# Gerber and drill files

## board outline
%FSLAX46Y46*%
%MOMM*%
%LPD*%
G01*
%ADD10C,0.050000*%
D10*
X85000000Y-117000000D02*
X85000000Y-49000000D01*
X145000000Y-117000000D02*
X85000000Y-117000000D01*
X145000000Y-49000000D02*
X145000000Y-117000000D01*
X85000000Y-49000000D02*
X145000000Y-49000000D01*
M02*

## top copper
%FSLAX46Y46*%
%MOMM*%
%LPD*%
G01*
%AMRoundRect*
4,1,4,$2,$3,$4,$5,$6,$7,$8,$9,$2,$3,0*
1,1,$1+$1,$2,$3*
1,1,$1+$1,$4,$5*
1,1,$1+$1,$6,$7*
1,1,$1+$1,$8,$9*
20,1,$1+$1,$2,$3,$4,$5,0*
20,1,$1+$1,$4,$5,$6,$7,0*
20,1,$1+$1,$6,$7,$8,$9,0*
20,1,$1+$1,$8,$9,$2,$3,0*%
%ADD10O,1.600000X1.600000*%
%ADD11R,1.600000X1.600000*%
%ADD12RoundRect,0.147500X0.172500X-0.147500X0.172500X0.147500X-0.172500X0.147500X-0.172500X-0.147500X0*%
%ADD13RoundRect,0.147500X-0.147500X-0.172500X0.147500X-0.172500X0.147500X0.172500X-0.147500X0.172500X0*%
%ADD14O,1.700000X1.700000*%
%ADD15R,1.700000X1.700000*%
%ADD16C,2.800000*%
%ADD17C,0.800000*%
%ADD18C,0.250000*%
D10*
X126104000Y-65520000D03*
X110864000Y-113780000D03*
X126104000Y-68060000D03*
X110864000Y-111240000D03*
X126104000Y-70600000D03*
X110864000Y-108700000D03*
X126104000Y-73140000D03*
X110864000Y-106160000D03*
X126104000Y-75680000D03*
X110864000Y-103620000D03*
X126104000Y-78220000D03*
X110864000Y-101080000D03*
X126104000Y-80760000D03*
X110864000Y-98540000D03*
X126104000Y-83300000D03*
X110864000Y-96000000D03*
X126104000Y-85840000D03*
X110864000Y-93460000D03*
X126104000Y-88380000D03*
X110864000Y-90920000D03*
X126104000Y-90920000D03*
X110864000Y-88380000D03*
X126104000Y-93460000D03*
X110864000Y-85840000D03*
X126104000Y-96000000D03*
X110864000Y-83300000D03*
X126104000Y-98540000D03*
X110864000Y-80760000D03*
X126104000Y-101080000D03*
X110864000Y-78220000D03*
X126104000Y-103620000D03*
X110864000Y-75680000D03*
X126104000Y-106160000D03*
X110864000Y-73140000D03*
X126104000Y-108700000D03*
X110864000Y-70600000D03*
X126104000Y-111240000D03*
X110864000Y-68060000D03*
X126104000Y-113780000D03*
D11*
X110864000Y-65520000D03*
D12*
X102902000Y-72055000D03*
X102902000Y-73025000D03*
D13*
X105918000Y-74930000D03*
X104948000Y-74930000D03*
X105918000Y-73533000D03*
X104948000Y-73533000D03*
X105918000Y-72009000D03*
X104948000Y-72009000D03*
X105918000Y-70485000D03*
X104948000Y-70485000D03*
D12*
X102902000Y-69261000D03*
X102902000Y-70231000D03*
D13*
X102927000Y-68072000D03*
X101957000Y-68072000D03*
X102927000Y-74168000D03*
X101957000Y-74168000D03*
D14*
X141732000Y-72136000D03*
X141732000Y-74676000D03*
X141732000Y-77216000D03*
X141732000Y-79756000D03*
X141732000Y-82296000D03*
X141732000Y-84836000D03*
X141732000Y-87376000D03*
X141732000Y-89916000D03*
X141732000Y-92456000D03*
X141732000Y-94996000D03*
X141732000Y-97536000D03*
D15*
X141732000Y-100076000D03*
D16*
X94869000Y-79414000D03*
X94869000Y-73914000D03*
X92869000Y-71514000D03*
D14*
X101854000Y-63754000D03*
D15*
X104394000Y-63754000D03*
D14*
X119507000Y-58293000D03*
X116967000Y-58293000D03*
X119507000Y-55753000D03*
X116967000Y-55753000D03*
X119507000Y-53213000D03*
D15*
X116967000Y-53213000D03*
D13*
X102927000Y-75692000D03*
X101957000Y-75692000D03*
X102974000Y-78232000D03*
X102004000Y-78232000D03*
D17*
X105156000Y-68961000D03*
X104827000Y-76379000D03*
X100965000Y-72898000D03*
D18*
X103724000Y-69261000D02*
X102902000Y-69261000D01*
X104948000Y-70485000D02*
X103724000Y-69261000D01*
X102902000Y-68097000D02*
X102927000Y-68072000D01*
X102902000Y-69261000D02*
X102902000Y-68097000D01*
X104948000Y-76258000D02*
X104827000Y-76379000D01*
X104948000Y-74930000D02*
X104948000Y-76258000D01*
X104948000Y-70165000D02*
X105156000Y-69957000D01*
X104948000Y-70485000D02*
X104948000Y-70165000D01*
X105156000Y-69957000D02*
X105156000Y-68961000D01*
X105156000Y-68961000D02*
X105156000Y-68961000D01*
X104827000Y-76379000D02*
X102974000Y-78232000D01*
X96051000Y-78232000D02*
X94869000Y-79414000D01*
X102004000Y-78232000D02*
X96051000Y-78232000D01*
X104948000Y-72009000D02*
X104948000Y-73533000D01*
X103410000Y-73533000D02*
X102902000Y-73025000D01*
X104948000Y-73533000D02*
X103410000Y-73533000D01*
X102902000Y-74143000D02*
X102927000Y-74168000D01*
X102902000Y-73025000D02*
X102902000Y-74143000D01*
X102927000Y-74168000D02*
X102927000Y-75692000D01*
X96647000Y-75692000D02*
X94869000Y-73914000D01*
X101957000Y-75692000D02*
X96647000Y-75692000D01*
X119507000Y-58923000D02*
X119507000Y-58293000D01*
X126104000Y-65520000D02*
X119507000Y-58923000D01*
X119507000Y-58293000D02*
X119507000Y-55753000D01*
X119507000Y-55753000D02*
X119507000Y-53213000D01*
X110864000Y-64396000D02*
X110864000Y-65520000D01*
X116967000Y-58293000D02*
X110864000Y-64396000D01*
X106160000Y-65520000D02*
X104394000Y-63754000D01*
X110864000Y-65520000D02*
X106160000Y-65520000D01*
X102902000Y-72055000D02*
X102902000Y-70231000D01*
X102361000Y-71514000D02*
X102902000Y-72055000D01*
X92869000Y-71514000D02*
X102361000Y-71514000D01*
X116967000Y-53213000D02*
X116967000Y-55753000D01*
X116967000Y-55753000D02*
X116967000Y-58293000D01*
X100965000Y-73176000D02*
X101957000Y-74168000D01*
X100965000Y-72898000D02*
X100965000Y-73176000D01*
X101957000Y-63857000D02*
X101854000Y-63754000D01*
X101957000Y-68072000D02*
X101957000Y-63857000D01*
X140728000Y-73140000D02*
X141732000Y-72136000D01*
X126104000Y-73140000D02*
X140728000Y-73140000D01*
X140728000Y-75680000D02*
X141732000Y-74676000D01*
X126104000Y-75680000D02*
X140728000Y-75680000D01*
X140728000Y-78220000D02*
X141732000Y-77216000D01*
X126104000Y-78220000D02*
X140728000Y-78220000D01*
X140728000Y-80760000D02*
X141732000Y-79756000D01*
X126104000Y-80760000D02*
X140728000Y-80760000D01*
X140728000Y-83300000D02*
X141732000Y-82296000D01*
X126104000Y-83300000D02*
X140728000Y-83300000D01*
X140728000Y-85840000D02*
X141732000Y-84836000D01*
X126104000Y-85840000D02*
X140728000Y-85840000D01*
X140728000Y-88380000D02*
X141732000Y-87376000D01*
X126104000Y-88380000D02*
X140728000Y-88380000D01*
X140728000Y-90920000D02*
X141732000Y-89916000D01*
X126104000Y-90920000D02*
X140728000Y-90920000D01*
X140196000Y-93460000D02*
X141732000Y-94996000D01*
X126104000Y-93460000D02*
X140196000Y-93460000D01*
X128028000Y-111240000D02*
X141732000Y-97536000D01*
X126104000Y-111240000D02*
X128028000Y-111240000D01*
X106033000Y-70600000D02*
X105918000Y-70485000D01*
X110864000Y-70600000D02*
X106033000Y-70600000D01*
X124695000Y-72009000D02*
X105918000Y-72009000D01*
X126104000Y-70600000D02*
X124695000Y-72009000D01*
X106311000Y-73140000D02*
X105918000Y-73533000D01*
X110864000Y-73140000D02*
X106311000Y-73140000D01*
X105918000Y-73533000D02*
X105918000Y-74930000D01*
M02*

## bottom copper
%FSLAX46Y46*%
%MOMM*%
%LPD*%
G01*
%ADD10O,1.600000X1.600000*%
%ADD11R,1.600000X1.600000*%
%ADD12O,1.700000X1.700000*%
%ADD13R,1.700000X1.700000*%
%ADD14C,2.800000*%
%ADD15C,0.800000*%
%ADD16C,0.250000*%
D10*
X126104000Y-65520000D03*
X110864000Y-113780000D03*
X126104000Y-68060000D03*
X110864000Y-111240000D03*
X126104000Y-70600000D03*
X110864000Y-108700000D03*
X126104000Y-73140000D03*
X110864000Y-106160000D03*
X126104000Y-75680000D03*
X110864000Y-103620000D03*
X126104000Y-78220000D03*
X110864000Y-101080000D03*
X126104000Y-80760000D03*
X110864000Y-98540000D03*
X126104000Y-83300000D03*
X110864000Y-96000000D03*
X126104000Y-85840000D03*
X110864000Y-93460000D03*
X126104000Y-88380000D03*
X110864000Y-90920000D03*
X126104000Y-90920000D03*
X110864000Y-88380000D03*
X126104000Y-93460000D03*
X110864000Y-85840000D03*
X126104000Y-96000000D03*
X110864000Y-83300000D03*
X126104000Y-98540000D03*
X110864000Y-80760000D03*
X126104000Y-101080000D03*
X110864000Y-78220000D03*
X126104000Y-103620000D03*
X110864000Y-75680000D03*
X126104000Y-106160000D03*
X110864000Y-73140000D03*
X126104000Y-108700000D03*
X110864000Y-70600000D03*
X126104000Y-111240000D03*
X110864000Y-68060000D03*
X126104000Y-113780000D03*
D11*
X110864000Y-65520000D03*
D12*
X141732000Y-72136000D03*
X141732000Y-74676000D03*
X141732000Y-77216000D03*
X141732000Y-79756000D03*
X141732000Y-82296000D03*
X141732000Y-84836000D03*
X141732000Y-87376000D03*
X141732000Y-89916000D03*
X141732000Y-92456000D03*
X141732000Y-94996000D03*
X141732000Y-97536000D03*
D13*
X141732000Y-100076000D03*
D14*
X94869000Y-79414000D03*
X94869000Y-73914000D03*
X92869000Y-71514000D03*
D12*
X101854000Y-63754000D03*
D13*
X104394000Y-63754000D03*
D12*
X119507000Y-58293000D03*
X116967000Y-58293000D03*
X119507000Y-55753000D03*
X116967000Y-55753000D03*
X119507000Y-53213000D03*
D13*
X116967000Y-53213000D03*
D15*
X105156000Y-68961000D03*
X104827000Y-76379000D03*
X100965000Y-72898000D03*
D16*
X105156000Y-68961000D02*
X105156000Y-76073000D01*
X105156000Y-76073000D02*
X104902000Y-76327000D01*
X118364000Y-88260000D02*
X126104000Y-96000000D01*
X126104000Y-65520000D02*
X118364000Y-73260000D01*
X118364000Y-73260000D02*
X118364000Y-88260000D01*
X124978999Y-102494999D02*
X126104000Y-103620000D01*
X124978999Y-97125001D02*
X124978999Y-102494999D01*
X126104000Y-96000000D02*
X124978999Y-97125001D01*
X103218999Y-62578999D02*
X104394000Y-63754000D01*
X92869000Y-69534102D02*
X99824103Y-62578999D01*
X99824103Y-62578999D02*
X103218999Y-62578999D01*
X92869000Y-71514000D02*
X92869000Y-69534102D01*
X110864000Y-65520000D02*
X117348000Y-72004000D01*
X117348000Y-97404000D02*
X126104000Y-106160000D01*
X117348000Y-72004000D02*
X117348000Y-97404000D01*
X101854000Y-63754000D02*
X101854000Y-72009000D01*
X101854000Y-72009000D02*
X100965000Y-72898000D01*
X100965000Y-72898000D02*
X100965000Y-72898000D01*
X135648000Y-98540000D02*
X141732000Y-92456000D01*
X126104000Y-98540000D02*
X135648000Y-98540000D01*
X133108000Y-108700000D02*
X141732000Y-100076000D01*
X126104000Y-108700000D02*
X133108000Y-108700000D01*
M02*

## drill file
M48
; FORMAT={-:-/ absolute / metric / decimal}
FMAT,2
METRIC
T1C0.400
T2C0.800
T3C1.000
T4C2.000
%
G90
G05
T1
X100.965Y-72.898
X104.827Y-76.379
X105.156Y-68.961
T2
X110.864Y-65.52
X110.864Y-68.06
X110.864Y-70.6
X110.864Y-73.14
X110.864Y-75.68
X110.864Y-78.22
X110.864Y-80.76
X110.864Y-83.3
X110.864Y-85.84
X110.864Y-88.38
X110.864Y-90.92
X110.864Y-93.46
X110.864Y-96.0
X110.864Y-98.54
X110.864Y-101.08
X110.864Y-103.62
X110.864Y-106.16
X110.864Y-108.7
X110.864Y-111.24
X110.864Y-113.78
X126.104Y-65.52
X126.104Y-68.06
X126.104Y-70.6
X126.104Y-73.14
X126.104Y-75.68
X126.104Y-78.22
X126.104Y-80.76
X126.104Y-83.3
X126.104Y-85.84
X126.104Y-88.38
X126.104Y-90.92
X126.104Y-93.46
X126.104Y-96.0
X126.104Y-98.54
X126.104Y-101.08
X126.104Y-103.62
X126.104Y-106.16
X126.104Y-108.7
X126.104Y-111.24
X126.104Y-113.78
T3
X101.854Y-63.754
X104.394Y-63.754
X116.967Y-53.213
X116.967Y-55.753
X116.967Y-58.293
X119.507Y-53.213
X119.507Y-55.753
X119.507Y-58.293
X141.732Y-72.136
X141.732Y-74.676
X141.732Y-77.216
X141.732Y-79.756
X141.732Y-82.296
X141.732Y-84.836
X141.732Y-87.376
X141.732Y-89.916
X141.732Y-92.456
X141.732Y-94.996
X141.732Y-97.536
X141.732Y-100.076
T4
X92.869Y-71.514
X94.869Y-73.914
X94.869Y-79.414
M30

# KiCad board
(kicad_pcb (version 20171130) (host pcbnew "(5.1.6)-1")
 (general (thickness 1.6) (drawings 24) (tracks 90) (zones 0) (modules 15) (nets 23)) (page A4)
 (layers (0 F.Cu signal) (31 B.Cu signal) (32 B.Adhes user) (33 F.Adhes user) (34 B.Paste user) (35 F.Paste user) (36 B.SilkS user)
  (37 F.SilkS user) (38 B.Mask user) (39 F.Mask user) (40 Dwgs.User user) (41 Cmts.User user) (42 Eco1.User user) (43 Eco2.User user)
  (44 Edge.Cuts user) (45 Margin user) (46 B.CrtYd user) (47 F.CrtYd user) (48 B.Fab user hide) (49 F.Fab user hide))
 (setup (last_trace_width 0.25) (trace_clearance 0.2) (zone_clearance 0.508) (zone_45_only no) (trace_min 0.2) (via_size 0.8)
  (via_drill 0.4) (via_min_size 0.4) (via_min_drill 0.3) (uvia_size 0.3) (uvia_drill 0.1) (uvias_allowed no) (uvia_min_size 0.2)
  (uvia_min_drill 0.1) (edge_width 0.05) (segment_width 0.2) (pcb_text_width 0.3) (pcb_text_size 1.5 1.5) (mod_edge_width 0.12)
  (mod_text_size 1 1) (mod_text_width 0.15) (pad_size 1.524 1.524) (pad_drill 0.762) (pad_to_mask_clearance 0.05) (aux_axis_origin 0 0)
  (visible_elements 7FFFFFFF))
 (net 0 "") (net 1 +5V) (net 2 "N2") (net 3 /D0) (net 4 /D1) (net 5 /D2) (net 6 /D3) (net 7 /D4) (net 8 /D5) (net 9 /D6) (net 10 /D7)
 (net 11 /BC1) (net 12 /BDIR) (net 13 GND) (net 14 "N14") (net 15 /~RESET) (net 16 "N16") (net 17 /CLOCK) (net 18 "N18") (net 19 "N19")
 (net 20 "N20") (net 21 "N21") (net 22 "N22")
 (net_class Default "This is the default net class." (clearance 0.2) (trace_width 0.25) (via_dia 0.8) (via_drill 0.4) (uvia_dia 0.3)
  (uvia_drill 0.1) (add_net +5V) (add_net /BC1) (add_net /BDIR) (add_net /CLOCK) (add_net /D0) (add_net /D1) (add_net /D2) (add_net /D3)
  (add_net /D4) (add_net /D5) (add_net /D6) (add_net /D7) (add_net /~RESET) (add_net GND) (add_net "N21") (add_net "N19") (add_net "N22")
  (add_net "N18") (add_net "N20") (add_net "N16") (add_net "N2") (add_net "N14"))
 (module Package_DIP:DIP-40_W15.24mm (layer F.Cu) (at 110.864 65.52)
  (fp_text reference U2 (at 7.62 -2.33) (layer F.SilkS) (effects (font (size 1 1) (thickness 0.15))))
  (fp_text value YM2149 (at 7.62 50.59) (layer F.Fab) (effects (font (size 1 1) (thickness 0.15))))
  (pad 40 thru_hole oval (at 15.24 0) (size 1.6 1.6) (drill 0.8) (layers *.Cu *.Mask) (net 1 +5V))
  (pad 20 thru_hole oval (at 0 48.26) (size 1.6 1.6) (drill 0.8) (layers *.Cu *.Mask))
  (pad 39 thru_hole oval (at 15.24 2.54) (size 1.6 1.6) (drill 0.8) (layers *.Cu *.Mask))
  (pad 19 thru_hole oval (at 0 45.72) (size 1.6 1.6) (drill 0.8) (layers *.Cu *.Mask))
  (pad 38 thru_hole oval (at 15.24 5.08) (size 1.6 1.6) (drill 0.8) (layers *.Cu *.Mask) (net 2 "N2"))
  (pad 18 thru_hole oval (at 0 43.18) (size 1.6 1.6) (drill 0.8) (layers *.Cu *.Mask))
  (pad 37 thru_hole oval (at 15.24 7.62) (size 1.6 1.6) (drill 0.8) (layers *.Cu *.Mask) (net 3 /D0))
  (pad 17 thru_hole oval (at 0 40.64) (size 1.6 1.6) (drill 0.8) (layers *.Cu *.Mask))
  (pad 36 thru_hole oval (at 15.24 10.16) (size 1.6 1.6) (drill 0.8) (layers *.Cu *.Mask) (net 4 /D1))
  (pad 16 thru_hole oval (at 0 38.1) (size 1.6 1.6) (drill 0.8) (layers *.Cu *.Mask))
  (pad 35 thru_hole oval (at 15.24 12.7) (size 1.6 1.6) (drill 0.8) (layers *.Cu *.Mask) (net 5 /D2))
  (pad 15 thru_hole oval (at 0 35.56) (size 1.6 1.6) (drill 0.8) (layers *.Cu *.Mask))
  (pad 34 thru_hole oval (at 15.24 15.24) (size 1.6 1.6) (drill 0.8) (layers *.Cu *.Mask) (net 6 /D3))
  (pad 14 thru_hole oval (at 0 33.02) (size 1.6 1.6) (drill 0.8) (layers *.Cu *.Mask))
  (pad 33 thru_hole oval (at 15.24 17.78) (size 1.6 1.6) (drill 0.8) (layers *.Cu *.Mask) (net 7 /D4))
  (pad 13 thru_hole oval (at 0 30.48) (size 1.6 1.6) (drill 0.8) (layers *.Cu *.Mask))
  (pad 32 thru_hole oval (at 15.24 20.32) (size 1.6 1.6) (drill 0.8) (layers *.Cu *.Mask) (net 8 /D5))
  (pad 12 thru_hole oval (at 0 27.94) (size 1.6 1.6) (drill 0.8) (layers *.Cu *.Mask))
  (pad 31 thru_hole oval (at 15.24 22.86) (size 1.6 1.6) (drill 0.8) (layers *.Cu *.Mask) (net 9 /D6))
  (pad 11 thru_hole oval (at 0 25.4) (size 1.6 1.6) (drill 0.8) (layers *.Cu *.Mask))
  (pad 30 thru_hole oval (at 15.24 25.4) (size 1.6 1.6) (drill 0.8) (layers *.Cu *.Mask) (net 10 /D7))
  (pad 10 thru_hole oval (at 0 22.86) (size 1.6 1.6) (drill 0.8) (layers *.Cu *.Mask))
  (pad 29 thru_hole oval (at 15.24 27.94) (size 1.6 1.6) (drill 0.8) (layers *.Cu *.Mask) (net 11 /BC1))
  (pad 9 thru_hole oval (at 0 20.32) (size 1.6 1.6) (drill 0.8) (layers *.Cu *.Mask))
  (pad 28 thru_hole oval (at 15.24 30.48) (size 1.6 1.6) (drill 0.8) (layers *.Cu *.Mask) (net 1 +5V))
  (pad 8 thru_hole oval (at 0 17.78) (size 1.6 1.6) (drill 0.8) (layers *.Cu *.Mask))
  (pad 27 thru_hole oval (at 15.24 33.02) (size 1.6 1.6) (drill 0.8) (layers *.Cu *.Mask) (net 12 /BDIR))
  (pad 7 thru_hole oval (at 0 15.24) (size 1.6 1.6) (drill 0.8) (layers *.Cu *.Mask))
  (pad 26 thru_hole oval (at 15.24 35.56) (size 1.6 1.6) (drill 0.8) (layers *.Cu *.Mask))
  (pad 6 thru_hole oval (at 0 12.7) (size 1.6 1.6) (drill 0.8) (layers *.Cu *.Mask))
  (pad 25 thru_hole oval (at 15.24 38.1) (size 1.6 1.6) (drill 0.8) (layers *.Cu *.Mask) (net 1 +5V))
  (pad 5 thru_hole oval (at 0 10.16) (size 1.6 1.6) (drill 0.8) (layers *.Cu *.Mask))
  (pad 24 thru_hole oval (at 15.24 40.64) (size 1.6 1.6) (drill 0.8) (layers *.Cu *.Mask) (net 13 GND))
  (pad 4 thru_hole oval (at 0 7.62) (size 1.6 1.6) (drill 0.8) (layers *.Cu *.Mask) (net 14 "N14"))
  (pad 23 thru_hole oval (at 15.24 43.18) (size 1.6 1.6) (drill 0.8) (layers *.Cu *.Mask) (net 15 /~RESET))
  (pad 3 thru_hole oval (at 0 5.08) (size 1.6 1.6) (drill 0.8) (layers *.Cu *.Mask) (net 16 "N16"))
  (pad 22 thru_hole oval (at 15.24 45.72) (size 1.6 1.6) (drill 0.8) (layers *.Cu *.Mask) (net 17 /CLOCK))
  (pad 2 thru_hole oval (at 0 2.54) (size 1.6 1.6) (drill 0.8) (layers *.Cu *.Mask))
  (pad 21 thru_hole oval (at 15.24 48.26) (size 1.6 1.6) (drill 0.8) (layers *.Cu *.Mask))
  (pad 1 thru_hole rect (at 0 0) (size 1.6 1.6) (drill 0.8) (layers *.Cu *.Mask) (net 13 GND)))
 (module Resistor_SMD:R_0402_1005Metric (layer F.Cu) (at 102.902 72.54 90)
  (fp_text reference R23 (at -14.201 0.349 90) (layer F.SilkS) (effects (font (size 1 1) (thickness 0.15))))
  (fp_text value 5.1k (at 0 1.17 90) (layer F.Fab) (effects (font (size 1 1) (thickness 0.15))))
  (pad 2 smd roundrect (at 0.485 0 90) (size 0.59 0.64) (layers F.Cu F.Paste F.Mask) (roundrect_rratio 0.25) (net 13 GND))
  (pad 1 smd roundrect (at -0.485 0 90) (size 0.59 0.64) (layers F.Cu F.Paste F.Mask) (roundrect_rratio 0.25) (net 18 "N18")))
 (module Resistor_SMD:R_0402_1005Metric (layer F.Cu) (at 105.433 74.93)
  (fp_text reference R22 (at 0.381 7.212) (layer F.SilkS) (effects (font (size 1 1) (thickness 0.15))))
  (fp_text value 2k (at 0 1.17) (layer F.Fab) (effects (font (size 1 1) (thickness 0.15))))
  (pad 2 smd roundrect (at 0.485 0) (size 0.59 0.64) (layers F.Cu F.Paste F.Mask) (roundrect_rratio 0.25) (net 14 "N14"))
  (pad 1 smd roundrect (at -0.485 0) (size 0.59 0.64) (layers F.Cu F.Paste F.Mask) (roundrect_rratio 0.25) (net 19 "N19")))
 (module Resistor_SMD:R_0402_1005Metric (layer F.Cu) (at 105.433 73.533)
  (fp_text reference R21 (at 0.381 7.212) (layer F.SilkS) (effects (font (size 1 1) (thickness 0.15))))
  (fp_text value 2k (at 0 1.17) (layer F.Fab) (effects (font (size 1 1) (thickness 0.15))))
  (pad 2 smd roundrect (at 0.485 0) (size 0.59 0.64) (layers F.Cu F.Paste F.Mask) (roundrect_rratio 0.25) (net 14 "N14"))
  (pad 1 smd roundrect (at -0.485 0) (size 0.59 0.64) (layers F.Cu F.Paste F.Mask) (roundrect_rratio 0.25) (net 18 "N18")))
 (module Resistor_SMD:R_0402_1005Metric (layer F.Cu) (at 105.433 72.009)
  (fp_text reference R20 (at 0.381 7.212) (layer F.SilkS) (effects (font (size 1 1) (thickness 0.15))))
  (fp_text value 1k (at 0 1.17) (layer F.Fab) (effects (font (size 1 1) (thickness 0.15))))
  (pad 2 smd roundrect (at 0.485 0) (size 0.59 0.64) (layers F.Cu F.Paste F.Mask) (roundrect_rratio 0.25) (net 2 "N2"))
  (pad 1 smd roundrect (at -0.485 0) (size 0.59 0.64) (layers F.Cu F.Paste F.Mask) (roundrect_rratio 0.25) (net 18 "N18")))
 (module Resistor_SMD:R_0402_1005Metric (layer F.Cu) (at 105.433 70.485)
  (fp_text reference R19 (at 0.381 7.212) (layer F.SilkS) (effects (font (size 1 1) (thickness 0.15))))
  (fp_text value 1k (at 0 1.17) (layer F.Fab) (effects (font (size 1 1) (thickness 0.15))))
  (pad 2 smd roundrect (at 0.485 0) (size 0.59 0.64) (layers F.Cu F.Paste F.Mask) (roundrect_rratio 0.25) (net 16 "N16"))
  (pad 1 smd roundrect (at -0.485 0) (size 0.59 0.64) (layers F.Cu F.Paste F.Mask) (roundrect_rratio 0.25) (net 19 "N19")))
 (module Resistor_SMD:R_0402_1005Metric (layer F.Cu) (at 102.902 69.746 90)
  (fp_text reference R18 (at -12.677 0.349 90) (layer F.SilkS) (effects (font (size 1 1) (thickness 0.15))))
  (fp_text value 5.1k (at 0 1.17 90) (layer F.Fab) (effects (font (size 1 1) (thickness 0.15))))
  (pad 2 smd roundrect (at 0.485 0 90) (size 0.59 0.64) (layers F.Cu F.Paste F.Mask) (roundrect_rratio 0.25) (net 19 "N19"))
  (pad 1 smd roundrect (at -0.485 0 90) (size 0.59 0.64) (layers F.Cu F.Paste F.Mask) (roundrect_rratio 0.25) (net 13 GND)))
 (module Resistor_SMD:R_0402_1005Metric (layer F.Cu) (at 102.442 68.072)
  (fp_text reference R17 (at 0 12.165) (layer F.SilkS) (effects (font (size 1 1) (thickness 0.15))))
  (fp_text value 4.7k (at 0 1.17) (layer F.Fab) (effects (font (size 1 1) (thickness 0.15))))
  (pad 2 smd roundrect (at 0.485 0) (size 0.59 0.64) (layers F.Cu F.Paste F.Mask) (roundrect_rratio 0.25) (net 19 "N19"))
  (pad 1 smd roundrect (at -0.485 0) (size 0.59 0.64) (layers F.Cu F.Paste F.Mask) (roundrect_rratio 0.25) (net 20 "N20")))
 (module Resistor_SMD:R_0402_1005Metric (layer F.Cu) (at 102.442 74.168)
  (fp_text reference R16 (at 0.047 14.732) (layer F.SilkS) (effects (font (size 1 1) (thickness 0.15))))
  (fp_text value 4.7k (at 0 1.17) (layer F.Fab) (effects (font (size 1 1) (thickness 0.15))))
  (pad 2 smd roundrect (at 0.485 0) (size 0.59 0.64) (layers F.Cu F.Paste F.Mask) (roundrect_rratio 0.25) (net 18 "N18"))
  (pad 1 smd roundrect (at -0.485 0) (size 0.59 0.64) (layers F.Cu F.Paste F.Mask) (roundrect_rratio 0.25) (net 20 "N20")))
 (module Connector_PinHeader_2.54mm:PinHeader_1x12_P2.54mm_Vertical (layer F.Cu) (at 141.732 100.076 180)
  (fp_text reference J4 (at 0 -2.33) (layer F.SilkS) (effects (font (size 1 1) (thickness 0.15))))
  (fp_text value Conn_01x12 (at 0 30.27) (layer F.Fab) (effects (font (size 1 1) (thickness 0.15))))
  (pad 12 thru_hole oval (at 0 27.94 180) (size 1.7 1.7) (drill 1) (layers *.Cu *.Mask) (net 3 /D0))
  (pad 11 thru_hole oval (at 0 25.4 180) (size 1.7 1.7) (drill 1) (layers *.Cu *.Mask) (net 4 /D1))
  (pad 10 thru_hole oval (at 0 22.86 180) (size 1.7 1.7) (drill 1) (layers *.Cu *.Mask) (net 5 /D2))
  (pad 9 thru_hole oval (at 0 20.32 180) (size 1.7 1.7) (drill 1) (layers *.Cu *.Mask) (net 6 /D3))
  (pad 8 thru_hole oval (at 0 17.78 180) (size 1.7 1.7) (drill 1) (layers *.Cu *.Mask) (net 7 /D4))
  (pad 7 thru_hole oval (at 0 15.24 180) (size 1.7 1.7) (drill 1) (layers *.Cu *.Mask) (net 8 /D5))
  (pad 6 thru_hole oval (at 0 12.7 180) (size 1.7 1.7) (drill 1) (layers *.Cu *.Mask) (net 9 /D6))
  (pad 5 thru_hole oval (at 0 10.16 180) (size 1.7 1.7) (drill 1) (layers *.Cu *.Mask) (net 10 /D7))
  (pad 4 thru_hole oval (at 0 7.62 180) (size 1.7 1.7) (drill 1) (layers *.Cu *.Mask) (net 12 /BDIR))
  (pad 3 thru_hole oval (at 0 5.08 180) (size 1.7 1.7) (drill 1) (layers *.Cu *.Mask) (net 11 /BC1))
  (pad 2 thru_hole oval (at 0 2.54 180) (size 1.7 1.7) (drill 1) (layers *.Cu *.Mask) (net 17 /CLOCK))
  (pad 1 thru_hole rect (at 0 0 180) (size 1.7 1.7) (drill 1) (layers *.Cu *.Mask) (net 15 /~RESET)))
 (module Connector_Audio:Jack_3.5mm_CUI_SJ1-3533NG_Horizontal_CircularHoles (layer F.Cu) (at 92.869 71.514)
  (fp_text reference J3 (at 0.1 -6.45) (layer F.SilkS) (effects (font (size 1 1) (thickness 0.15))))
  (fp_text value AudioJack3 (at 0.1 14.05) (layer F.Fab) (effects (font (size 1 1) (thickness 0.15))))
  (pad R thru_hole circle (at 2 7.9) (size 2.8 2.8) (drill 2) (layers *.Cu *.Mask) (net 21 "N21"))
  (pad T thru_hole circle (at 2 2.4) (size 2.8 2.8) (drill 2) (layers *.Cu *.Mask) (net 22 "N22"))
  (pad S thru_hole circle (at 0 0) (size 2.8 2.8) (drill 2) (layers *.Cu *.Mask) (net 13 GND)))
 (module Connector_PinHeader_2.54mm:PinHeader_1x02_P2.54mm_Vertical (layer F.Cu) (at 104.394 63.754 270)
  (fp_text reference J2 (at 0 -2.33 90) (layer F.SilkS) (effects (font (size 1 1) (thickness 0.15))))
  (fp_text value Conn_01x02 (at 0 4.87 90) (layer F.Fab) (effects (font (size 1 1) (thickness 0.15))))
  (pad 2 thru_hole oval (at 0 2.54 270) (size 1.7 1.7) (drill 1) (layers *.Cu *.Mask) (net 20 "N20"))
  (pad 1 thru_hole rect (at 0 0 270) (size 1.7 1.7) (drill 1) (layers *.Cu *.Mask) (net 13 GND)))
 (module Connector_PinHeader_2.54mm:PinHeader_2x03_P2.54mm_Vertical (layer F.Cu) (at 116.967 53.213)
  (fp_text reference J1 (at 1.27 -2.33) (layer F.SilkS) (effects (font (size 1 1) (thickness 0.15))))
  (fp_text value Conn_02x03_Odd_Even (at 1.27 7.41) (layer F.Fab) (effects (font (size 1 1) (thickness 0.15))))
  (pad 6 thru_hole oval (at 2.54 5.08) (size 1.7 1.7) (drill 1) (layers *.Cu *.Mask) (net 1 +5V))
  (pad 5 thru_hole oval (at 0 5.08) (size 1.7 1.7) (drill 1) (layers *.Cu *.Mask) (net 13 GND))
  (pad 4 thru_hole oval (at 2.54 2.54) (size 1.7 1.7) (drill 1) (layers *.Cu *.Mask) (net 1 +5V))
  (pad 3 thru_hole oval (at 0 2.54) (size 1.7 1.7) (drill 1) (layers *.Cu *.Mask) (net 13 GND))
  (pad 2 thru_hole oval (at 2.54 0) (size 1.7 1.7) (drill 1) (layers *.Cu *.Mask) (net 1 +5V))
  (pad 1 thru_hole rect (at 0 0) (size 1.7 1.7) (drill 1) (layers *.Cu *.Mask) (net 13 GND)))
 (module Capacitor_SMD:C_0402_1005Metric (layer F.Cu) (at 102.442 75.692)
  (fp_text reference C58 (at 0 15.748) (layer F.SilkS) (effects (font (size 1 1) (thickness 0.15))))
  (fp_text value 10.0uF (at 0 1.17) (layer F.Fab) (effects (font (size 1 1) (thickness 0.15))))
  (pad 2 smd roundrect (at 0.485 0) (size 0.59 0.64) (layers F.Cu F.Paste F.Mask) (roundrect_rratio 0.25) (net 18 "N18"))
  (pad 1 smd roundrect (at -0.485 0) (size 0.59 0.64) (layers F.Cu F.Paste F.Mask) (roundrect_rratio 0.25) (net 22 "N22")))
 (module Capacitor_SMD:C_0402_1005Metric (layer F.Cu) (at 102.489 78.232)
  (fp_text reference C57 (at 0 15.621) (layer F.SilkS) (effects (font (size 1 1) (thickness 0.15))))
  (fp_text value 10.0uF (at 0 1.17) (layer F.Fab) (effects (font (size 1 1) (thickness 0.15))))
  (pad 2 smd roundrect (at 0.485 0) (size 0.59 0.64) (layers F.Cu F.Paste F.Mask) (roundrect_rratio 0.25) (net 19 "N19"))
  (pad 1 smd roundrect (at -0.485 0) (size 0.59 0.64) (layers F.Cu F.Paste F.Mask) (roundrect_rratio 0.25) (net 21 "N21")))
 (gr_line (start 85 117) (end 85 49) (layer Edge.Cuts) (width 0.05))
 (gr_line (start 145 117) (end 85 117) (layer Edge.Cuts) (width 0.05))
 (gr_line (start 145 49) (end 145 117) (layer Edge.Cuts) (width 0.05))
 (gr_line (start 85 49) (end 145 49) (layer Edge.Cuts) (width 0.05))
 (segment (start 103.724 69.261) (end 102.902 69.261) (width 0.25) (layer F.Cu) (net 19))
 (segment (start 104.948 70.485) (end 103.724 69.261) (width 0.25) (layer F.Cu) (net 19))
 (segment (start 102.902 68.097) (end 102.927 68.072) (width 0.25) (layer F.Cu) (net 19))
 (segment (start 102.902 69.261) (end 102.902 68.097) (width 0.25) (layer F.Cu) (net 19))
 (segment (start 104.948 76.258) (end 104.827 76.379) (width 0.25) (layer F.Cu) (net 19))
 (segment (start 104.948 74.93) (end 104.948 76.258) (width 0.25) (layer F.Cu) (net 19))
 (segment (start 104.948 70.165) (end 105.156 69.957) (width 0.25) (layer F.Cu) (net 19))
 (segment (start 104.948 70.485) (end 104.948 70.165) (width 0.25) (layer F.Cu) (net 19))
 (segment (start 105.156 69.957) (end 105.156 68.961) (width 0.25) (layer F.Cu) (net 19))
 (segment (start 105.156 68.961) (end 105.156 68.961) (width 0.25) (layer F.Cu) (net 19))
 (via (at 105.156 68.961) (size 0.8) (drill 0.4) (layers F.Cu B.Cu) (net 19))
 (segment (start 105.156 68.961) (end 105.156 76.073) (width 0.25) (layer B.Cu) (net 19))
 (segment (start 105.156 76.073) (end 104.902 76.327) (width 0.25) (layer B.Cu) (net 19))
 (segment (start 104.827 76.379) (end 102.974 78.232) (width 0.25) (layer F.Cu) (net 19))
 (via (at 104.827 76.379) (size 0.8) (drill 0.4) (layers F.Cu B.Cu) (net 19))
 (segment (start 96.051 78.232) (end 94.869 79.414) (width 0.25) (layer F.Cu) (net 21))
 (segment (start 102.004 78.232) (end 96.051 78.232) (width 0.25) (layer F.Cu) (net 21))
 (segment (start 104.948 72.009) (end 104.948 73.533) (width 0.25) (layer F.Cu) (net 18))
 (segment (start 103.41 73.533) (end 102.902 73.025) (width 0.25) (layer F.Cu) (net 18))
 (segment (start 104.948 73.533) (end 103.41 73.533) (width 0.25) (layer F.Cu) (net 18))
 (segment (start 102.902 74.143) (end 102.927 74.168) (width 0.25) (layer F.Cu) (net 18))
 (segment (start 102.902 73.025) (end 102.902 74.143) (width 0.25) (layer F.Cu) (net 18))
 (segment (start 102.927 74.168) (end 102.927 75.692) (width 0.25) (layer F.Cu) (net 18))
 (segment (start 96.647 75.692) (end 94.869 73.914) (width 0.25) (layer F.Cu) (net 22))
 (segment (start 101.957 75.692) (end 96.647 75.692) (width 0.25) (layer F.Cu) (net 22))
 (segment (start 119.507 58.923) (end 119.507 58.293) (width 0.25) (layer F.Cu) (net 1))
 (segment (start 126.104 65.52) (end 119.507 58.923) (width 0.25) (layer F.Cu) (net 1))
 (segment (start 119.507 58.293) (end 119.507 55.753) (width 0.25) (layer F.Cu) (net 1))
 (segment (start 119.507 55.753) (end 119.507 53.213) (width 0.25) (layer F.Cu) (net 1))
 (segment (start 118.364 88.26) (end 126.104 96) (width 0.25) (layer B.Cu) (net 1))
 (segment (start 126.104 65.52) (end 118.364 73.26) (width 0.25) (layer B.Cu) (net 1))
 (segment (start 118.364 73.26) (end 118.364 88.26) (width 0.25) (layer B.Cu) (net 1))
 (segment (start 124.978999 102.494999) (end 126.104 103.62) (width 0.25) (layer B.Cu) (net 1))
 (segment (start 124.978999 97.125001) (end 124.978999 102.494999) (width 0.25) (layer B.Cu) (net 1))
 (segment (start 126.104 96) (end 124.978999 97.125001) (width 0.25) (layer B.Cu) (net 1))
 (segment (start 110.864 64.396) (end 110.864 65.52) (width 0.25) (layer F.Cu) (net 13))
 (segment (start 116.967 58.293) (end 110.864 64.396) (width 0.25) (layer F.Cu) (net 13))
 (segment (start 106.16 65.52) (end 104.394 63.754) (width 0.25) (layer F.Cu) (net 13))
 (segment (start 110.864 65.52) (end 106.16 65.52) (width 0.25) (layer F.Cu) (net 13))
 (segment (start 103.218999 62.578999) (end 104.394 63.754) (width 0.25) (layer B.Cu) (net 13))
 (segment (start 92.869 69.534102) (end 99.824103 62.578999) (width 0.25) (layer B.Cu) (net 13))
 (segment (start 99.824103 62.578999) (end 103.218999 62.578999) (width 0.25) (layer B.Cu) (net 13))
 (segment (start 92.869 71.514) (end 92.869 69.534102) (width 0.25) (layer B.Cu) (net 13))
 (segment (start 102.902 72.055) (end 102.902 70.231) (width 0.25) (layer F.Cu) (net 13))
 (segment (start 110.864 65.52) (end 117.348 72.004) (width 0.25) (layer B.Cu) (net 13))
 (segment (start 117.348 97.404) (end 126.104 106.16) (width 0.25) (layer B.Cu) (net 13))
 (segment (start 117.348 72.004) (end 117.348 97.404) (width 0.25) (layer B.Cu) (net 13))
 (segment (start 102.361 71.514) (end 102.902 72.055) (width 0.25) (layer F.Cu) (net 13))
 (segment (start 92.869 71.514) (end 102.361 71.514) (width 0.25) (layer F.Cu) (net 13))
 (segment (start 116.967 53.213) (end 116.967 55.753) (width 0.25) (layer F.Cu) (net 13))
 (segment (start 116.967 55.753) (end 116.967 58.293) (width 0.25) (layer F.Cu) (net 13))
 (segment (start 101.854 63.754) (end 101.854 72.009) (width 0.25) (layer B.Cu) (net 20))
 (segment (start 101.854 72.009) (end 100.965 72.898) (width 0.25) (layer B.Cu) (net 20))
 (segment (start 100.965 72.898) (end 100.965 72.898) (width 0.25) (layer B.Cu) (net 20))
 (via (at 100.965 72.898) (size 0.8) (drill 0.4) (layers F.Cu B.Cu) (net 20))
 (segment (start 100.965 73.176) (end 101.957 74.168) (width 0.25) (layer F.Cu) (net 20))
 (segment (start 100.965 72.898) (end 100.965 73.176) (width 0.25) (layer F.Cu) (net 20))
 (segment (start 101.957 63.857) (end 101.854 63.754) (width 0.25) (layer F.Cu) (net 20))
 (segment (start 101.957 68.072) (end 101.957 63.857) (width 0.25) (layer F.Cu) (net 20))
 (segment (start 140.728 73.14) (end 141.732 72.136) (width 0.25) (layer F.Cu) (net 3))
 (segment (start 126.104 73.14) (end 140.728 73.14) (width 0.25) (layer F.Cu) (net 3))
 (segment (start 140.728 75.68) (end 141.732 74.676) (width 0.25) (layer F.Cu) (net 4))
 (segment (start 126.104 75.68) (end 140.728 75.68) (width 0.25) (layer F.Cu) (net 4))
 (segment (start 140.728 78.22) (end 141.732 77.216) (width 0.25) (layer F.Cu) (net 5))
 (segment (start 126.104 78.22) (end 140.728 78.22) (width 0.25) (layer F.Cu) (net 5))
 (segment (start 140.728 80.76) (end 141.732 79.756) (width 0.25) (layer F.Cu) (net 6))
 (segment (start 126.104 80.76) (end 140.728 80.76) (width 0.25) (layer F.Cu) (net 6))
 (segment (start 140.728 83.3) (end 141.732 82.296) (width 0.25) (layer F.Cu) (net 7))
 (segment (start 126.104 83.3) (end 140.728 83.3) (width 0.25) (layer F.Cu) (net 7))
 (segment (start 140.728 85.84) (end 141.732 84.836) (width 0.25) (layer F.Cu) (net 8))
 (segment (start 126.104 85.84) (end 140.728 85.84) (width 0.25) (layer F.Cu) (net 8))
 (segment (start 140.728 88.38) (end 141.732 87.376) (width 0.25) (layer F.Cu) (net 9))
 (segment (start 126.104 88.38) (end 140.728 88.38) (width 0.25) (layer F.Cu) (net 9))
 (segment (start 140.728 90.92) (end 141.732 89.916) (width 0.25) (layer F.Cu) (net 10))
 (segment (start 126.104 90.92) (end 140.728 90.92) (width 0.25) (layer F.Cu) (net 10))
 (segment (start 135.648 98.54) (end 141.732 92.456) (width 0.25) (layer B.Cu) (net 12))
 (segment (start 126.104 98.54) (end 135.648 98.54) (width 0.25) (layer B.Cu) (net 12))
 (segment (start 140.196 93.46) (end 141.732 94.996) (width 0.25) (layer F.Cu) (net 11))
 (segment (start 126.104 93.46) (end 140.196 93.46) (width 0.25) (layer F.Cu) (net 11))
 (segment (start 128.028 111.24) (end 141.732 97.536) (width 0.25) (layer F.Cu) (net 17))
 (segment (start 126.104 111.24) (end 128.028 111.24) (width 0.25) (layer F.Cu) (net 17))
 (segment (start 133.108 108.7) (end 141.732 100.076) (width 0.25) (layer B.Cu) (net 15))
 (segment (start 126.104 108.7) (end 133.108 108.7) (width 0.25) (layer B.Cu) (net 15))
 (segment (start 106.033 70.6) (end 105.918 70.485) (width 0.25) (layer F.Cu) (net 16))
 (segment (start 110.864 70.6) (end 106.033 70.6) (width 0.25) (layer F.Cu) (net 16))
 (segment (start 124.695 72.009) (end 105.918 72.009) (width 0.25) (layer F.Cu) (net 2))
 (segment (start 126.104 70.6) (end 124.695 72.009) (width 0.25) (layer F.Cu) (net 2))
 (segment (start 106.311 73.14) (end 105.918 73.533) (width 0.25) (layer F.Cu) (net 14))
 (segment (start 110.864 73.14) (end 106.311 73.14) (width 0.25) (layer F.Cu) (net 14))
 (segment (start 105.918 73.533) (end 105.918 74.93) (width 0.25) (layer F.Cu) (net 14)))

